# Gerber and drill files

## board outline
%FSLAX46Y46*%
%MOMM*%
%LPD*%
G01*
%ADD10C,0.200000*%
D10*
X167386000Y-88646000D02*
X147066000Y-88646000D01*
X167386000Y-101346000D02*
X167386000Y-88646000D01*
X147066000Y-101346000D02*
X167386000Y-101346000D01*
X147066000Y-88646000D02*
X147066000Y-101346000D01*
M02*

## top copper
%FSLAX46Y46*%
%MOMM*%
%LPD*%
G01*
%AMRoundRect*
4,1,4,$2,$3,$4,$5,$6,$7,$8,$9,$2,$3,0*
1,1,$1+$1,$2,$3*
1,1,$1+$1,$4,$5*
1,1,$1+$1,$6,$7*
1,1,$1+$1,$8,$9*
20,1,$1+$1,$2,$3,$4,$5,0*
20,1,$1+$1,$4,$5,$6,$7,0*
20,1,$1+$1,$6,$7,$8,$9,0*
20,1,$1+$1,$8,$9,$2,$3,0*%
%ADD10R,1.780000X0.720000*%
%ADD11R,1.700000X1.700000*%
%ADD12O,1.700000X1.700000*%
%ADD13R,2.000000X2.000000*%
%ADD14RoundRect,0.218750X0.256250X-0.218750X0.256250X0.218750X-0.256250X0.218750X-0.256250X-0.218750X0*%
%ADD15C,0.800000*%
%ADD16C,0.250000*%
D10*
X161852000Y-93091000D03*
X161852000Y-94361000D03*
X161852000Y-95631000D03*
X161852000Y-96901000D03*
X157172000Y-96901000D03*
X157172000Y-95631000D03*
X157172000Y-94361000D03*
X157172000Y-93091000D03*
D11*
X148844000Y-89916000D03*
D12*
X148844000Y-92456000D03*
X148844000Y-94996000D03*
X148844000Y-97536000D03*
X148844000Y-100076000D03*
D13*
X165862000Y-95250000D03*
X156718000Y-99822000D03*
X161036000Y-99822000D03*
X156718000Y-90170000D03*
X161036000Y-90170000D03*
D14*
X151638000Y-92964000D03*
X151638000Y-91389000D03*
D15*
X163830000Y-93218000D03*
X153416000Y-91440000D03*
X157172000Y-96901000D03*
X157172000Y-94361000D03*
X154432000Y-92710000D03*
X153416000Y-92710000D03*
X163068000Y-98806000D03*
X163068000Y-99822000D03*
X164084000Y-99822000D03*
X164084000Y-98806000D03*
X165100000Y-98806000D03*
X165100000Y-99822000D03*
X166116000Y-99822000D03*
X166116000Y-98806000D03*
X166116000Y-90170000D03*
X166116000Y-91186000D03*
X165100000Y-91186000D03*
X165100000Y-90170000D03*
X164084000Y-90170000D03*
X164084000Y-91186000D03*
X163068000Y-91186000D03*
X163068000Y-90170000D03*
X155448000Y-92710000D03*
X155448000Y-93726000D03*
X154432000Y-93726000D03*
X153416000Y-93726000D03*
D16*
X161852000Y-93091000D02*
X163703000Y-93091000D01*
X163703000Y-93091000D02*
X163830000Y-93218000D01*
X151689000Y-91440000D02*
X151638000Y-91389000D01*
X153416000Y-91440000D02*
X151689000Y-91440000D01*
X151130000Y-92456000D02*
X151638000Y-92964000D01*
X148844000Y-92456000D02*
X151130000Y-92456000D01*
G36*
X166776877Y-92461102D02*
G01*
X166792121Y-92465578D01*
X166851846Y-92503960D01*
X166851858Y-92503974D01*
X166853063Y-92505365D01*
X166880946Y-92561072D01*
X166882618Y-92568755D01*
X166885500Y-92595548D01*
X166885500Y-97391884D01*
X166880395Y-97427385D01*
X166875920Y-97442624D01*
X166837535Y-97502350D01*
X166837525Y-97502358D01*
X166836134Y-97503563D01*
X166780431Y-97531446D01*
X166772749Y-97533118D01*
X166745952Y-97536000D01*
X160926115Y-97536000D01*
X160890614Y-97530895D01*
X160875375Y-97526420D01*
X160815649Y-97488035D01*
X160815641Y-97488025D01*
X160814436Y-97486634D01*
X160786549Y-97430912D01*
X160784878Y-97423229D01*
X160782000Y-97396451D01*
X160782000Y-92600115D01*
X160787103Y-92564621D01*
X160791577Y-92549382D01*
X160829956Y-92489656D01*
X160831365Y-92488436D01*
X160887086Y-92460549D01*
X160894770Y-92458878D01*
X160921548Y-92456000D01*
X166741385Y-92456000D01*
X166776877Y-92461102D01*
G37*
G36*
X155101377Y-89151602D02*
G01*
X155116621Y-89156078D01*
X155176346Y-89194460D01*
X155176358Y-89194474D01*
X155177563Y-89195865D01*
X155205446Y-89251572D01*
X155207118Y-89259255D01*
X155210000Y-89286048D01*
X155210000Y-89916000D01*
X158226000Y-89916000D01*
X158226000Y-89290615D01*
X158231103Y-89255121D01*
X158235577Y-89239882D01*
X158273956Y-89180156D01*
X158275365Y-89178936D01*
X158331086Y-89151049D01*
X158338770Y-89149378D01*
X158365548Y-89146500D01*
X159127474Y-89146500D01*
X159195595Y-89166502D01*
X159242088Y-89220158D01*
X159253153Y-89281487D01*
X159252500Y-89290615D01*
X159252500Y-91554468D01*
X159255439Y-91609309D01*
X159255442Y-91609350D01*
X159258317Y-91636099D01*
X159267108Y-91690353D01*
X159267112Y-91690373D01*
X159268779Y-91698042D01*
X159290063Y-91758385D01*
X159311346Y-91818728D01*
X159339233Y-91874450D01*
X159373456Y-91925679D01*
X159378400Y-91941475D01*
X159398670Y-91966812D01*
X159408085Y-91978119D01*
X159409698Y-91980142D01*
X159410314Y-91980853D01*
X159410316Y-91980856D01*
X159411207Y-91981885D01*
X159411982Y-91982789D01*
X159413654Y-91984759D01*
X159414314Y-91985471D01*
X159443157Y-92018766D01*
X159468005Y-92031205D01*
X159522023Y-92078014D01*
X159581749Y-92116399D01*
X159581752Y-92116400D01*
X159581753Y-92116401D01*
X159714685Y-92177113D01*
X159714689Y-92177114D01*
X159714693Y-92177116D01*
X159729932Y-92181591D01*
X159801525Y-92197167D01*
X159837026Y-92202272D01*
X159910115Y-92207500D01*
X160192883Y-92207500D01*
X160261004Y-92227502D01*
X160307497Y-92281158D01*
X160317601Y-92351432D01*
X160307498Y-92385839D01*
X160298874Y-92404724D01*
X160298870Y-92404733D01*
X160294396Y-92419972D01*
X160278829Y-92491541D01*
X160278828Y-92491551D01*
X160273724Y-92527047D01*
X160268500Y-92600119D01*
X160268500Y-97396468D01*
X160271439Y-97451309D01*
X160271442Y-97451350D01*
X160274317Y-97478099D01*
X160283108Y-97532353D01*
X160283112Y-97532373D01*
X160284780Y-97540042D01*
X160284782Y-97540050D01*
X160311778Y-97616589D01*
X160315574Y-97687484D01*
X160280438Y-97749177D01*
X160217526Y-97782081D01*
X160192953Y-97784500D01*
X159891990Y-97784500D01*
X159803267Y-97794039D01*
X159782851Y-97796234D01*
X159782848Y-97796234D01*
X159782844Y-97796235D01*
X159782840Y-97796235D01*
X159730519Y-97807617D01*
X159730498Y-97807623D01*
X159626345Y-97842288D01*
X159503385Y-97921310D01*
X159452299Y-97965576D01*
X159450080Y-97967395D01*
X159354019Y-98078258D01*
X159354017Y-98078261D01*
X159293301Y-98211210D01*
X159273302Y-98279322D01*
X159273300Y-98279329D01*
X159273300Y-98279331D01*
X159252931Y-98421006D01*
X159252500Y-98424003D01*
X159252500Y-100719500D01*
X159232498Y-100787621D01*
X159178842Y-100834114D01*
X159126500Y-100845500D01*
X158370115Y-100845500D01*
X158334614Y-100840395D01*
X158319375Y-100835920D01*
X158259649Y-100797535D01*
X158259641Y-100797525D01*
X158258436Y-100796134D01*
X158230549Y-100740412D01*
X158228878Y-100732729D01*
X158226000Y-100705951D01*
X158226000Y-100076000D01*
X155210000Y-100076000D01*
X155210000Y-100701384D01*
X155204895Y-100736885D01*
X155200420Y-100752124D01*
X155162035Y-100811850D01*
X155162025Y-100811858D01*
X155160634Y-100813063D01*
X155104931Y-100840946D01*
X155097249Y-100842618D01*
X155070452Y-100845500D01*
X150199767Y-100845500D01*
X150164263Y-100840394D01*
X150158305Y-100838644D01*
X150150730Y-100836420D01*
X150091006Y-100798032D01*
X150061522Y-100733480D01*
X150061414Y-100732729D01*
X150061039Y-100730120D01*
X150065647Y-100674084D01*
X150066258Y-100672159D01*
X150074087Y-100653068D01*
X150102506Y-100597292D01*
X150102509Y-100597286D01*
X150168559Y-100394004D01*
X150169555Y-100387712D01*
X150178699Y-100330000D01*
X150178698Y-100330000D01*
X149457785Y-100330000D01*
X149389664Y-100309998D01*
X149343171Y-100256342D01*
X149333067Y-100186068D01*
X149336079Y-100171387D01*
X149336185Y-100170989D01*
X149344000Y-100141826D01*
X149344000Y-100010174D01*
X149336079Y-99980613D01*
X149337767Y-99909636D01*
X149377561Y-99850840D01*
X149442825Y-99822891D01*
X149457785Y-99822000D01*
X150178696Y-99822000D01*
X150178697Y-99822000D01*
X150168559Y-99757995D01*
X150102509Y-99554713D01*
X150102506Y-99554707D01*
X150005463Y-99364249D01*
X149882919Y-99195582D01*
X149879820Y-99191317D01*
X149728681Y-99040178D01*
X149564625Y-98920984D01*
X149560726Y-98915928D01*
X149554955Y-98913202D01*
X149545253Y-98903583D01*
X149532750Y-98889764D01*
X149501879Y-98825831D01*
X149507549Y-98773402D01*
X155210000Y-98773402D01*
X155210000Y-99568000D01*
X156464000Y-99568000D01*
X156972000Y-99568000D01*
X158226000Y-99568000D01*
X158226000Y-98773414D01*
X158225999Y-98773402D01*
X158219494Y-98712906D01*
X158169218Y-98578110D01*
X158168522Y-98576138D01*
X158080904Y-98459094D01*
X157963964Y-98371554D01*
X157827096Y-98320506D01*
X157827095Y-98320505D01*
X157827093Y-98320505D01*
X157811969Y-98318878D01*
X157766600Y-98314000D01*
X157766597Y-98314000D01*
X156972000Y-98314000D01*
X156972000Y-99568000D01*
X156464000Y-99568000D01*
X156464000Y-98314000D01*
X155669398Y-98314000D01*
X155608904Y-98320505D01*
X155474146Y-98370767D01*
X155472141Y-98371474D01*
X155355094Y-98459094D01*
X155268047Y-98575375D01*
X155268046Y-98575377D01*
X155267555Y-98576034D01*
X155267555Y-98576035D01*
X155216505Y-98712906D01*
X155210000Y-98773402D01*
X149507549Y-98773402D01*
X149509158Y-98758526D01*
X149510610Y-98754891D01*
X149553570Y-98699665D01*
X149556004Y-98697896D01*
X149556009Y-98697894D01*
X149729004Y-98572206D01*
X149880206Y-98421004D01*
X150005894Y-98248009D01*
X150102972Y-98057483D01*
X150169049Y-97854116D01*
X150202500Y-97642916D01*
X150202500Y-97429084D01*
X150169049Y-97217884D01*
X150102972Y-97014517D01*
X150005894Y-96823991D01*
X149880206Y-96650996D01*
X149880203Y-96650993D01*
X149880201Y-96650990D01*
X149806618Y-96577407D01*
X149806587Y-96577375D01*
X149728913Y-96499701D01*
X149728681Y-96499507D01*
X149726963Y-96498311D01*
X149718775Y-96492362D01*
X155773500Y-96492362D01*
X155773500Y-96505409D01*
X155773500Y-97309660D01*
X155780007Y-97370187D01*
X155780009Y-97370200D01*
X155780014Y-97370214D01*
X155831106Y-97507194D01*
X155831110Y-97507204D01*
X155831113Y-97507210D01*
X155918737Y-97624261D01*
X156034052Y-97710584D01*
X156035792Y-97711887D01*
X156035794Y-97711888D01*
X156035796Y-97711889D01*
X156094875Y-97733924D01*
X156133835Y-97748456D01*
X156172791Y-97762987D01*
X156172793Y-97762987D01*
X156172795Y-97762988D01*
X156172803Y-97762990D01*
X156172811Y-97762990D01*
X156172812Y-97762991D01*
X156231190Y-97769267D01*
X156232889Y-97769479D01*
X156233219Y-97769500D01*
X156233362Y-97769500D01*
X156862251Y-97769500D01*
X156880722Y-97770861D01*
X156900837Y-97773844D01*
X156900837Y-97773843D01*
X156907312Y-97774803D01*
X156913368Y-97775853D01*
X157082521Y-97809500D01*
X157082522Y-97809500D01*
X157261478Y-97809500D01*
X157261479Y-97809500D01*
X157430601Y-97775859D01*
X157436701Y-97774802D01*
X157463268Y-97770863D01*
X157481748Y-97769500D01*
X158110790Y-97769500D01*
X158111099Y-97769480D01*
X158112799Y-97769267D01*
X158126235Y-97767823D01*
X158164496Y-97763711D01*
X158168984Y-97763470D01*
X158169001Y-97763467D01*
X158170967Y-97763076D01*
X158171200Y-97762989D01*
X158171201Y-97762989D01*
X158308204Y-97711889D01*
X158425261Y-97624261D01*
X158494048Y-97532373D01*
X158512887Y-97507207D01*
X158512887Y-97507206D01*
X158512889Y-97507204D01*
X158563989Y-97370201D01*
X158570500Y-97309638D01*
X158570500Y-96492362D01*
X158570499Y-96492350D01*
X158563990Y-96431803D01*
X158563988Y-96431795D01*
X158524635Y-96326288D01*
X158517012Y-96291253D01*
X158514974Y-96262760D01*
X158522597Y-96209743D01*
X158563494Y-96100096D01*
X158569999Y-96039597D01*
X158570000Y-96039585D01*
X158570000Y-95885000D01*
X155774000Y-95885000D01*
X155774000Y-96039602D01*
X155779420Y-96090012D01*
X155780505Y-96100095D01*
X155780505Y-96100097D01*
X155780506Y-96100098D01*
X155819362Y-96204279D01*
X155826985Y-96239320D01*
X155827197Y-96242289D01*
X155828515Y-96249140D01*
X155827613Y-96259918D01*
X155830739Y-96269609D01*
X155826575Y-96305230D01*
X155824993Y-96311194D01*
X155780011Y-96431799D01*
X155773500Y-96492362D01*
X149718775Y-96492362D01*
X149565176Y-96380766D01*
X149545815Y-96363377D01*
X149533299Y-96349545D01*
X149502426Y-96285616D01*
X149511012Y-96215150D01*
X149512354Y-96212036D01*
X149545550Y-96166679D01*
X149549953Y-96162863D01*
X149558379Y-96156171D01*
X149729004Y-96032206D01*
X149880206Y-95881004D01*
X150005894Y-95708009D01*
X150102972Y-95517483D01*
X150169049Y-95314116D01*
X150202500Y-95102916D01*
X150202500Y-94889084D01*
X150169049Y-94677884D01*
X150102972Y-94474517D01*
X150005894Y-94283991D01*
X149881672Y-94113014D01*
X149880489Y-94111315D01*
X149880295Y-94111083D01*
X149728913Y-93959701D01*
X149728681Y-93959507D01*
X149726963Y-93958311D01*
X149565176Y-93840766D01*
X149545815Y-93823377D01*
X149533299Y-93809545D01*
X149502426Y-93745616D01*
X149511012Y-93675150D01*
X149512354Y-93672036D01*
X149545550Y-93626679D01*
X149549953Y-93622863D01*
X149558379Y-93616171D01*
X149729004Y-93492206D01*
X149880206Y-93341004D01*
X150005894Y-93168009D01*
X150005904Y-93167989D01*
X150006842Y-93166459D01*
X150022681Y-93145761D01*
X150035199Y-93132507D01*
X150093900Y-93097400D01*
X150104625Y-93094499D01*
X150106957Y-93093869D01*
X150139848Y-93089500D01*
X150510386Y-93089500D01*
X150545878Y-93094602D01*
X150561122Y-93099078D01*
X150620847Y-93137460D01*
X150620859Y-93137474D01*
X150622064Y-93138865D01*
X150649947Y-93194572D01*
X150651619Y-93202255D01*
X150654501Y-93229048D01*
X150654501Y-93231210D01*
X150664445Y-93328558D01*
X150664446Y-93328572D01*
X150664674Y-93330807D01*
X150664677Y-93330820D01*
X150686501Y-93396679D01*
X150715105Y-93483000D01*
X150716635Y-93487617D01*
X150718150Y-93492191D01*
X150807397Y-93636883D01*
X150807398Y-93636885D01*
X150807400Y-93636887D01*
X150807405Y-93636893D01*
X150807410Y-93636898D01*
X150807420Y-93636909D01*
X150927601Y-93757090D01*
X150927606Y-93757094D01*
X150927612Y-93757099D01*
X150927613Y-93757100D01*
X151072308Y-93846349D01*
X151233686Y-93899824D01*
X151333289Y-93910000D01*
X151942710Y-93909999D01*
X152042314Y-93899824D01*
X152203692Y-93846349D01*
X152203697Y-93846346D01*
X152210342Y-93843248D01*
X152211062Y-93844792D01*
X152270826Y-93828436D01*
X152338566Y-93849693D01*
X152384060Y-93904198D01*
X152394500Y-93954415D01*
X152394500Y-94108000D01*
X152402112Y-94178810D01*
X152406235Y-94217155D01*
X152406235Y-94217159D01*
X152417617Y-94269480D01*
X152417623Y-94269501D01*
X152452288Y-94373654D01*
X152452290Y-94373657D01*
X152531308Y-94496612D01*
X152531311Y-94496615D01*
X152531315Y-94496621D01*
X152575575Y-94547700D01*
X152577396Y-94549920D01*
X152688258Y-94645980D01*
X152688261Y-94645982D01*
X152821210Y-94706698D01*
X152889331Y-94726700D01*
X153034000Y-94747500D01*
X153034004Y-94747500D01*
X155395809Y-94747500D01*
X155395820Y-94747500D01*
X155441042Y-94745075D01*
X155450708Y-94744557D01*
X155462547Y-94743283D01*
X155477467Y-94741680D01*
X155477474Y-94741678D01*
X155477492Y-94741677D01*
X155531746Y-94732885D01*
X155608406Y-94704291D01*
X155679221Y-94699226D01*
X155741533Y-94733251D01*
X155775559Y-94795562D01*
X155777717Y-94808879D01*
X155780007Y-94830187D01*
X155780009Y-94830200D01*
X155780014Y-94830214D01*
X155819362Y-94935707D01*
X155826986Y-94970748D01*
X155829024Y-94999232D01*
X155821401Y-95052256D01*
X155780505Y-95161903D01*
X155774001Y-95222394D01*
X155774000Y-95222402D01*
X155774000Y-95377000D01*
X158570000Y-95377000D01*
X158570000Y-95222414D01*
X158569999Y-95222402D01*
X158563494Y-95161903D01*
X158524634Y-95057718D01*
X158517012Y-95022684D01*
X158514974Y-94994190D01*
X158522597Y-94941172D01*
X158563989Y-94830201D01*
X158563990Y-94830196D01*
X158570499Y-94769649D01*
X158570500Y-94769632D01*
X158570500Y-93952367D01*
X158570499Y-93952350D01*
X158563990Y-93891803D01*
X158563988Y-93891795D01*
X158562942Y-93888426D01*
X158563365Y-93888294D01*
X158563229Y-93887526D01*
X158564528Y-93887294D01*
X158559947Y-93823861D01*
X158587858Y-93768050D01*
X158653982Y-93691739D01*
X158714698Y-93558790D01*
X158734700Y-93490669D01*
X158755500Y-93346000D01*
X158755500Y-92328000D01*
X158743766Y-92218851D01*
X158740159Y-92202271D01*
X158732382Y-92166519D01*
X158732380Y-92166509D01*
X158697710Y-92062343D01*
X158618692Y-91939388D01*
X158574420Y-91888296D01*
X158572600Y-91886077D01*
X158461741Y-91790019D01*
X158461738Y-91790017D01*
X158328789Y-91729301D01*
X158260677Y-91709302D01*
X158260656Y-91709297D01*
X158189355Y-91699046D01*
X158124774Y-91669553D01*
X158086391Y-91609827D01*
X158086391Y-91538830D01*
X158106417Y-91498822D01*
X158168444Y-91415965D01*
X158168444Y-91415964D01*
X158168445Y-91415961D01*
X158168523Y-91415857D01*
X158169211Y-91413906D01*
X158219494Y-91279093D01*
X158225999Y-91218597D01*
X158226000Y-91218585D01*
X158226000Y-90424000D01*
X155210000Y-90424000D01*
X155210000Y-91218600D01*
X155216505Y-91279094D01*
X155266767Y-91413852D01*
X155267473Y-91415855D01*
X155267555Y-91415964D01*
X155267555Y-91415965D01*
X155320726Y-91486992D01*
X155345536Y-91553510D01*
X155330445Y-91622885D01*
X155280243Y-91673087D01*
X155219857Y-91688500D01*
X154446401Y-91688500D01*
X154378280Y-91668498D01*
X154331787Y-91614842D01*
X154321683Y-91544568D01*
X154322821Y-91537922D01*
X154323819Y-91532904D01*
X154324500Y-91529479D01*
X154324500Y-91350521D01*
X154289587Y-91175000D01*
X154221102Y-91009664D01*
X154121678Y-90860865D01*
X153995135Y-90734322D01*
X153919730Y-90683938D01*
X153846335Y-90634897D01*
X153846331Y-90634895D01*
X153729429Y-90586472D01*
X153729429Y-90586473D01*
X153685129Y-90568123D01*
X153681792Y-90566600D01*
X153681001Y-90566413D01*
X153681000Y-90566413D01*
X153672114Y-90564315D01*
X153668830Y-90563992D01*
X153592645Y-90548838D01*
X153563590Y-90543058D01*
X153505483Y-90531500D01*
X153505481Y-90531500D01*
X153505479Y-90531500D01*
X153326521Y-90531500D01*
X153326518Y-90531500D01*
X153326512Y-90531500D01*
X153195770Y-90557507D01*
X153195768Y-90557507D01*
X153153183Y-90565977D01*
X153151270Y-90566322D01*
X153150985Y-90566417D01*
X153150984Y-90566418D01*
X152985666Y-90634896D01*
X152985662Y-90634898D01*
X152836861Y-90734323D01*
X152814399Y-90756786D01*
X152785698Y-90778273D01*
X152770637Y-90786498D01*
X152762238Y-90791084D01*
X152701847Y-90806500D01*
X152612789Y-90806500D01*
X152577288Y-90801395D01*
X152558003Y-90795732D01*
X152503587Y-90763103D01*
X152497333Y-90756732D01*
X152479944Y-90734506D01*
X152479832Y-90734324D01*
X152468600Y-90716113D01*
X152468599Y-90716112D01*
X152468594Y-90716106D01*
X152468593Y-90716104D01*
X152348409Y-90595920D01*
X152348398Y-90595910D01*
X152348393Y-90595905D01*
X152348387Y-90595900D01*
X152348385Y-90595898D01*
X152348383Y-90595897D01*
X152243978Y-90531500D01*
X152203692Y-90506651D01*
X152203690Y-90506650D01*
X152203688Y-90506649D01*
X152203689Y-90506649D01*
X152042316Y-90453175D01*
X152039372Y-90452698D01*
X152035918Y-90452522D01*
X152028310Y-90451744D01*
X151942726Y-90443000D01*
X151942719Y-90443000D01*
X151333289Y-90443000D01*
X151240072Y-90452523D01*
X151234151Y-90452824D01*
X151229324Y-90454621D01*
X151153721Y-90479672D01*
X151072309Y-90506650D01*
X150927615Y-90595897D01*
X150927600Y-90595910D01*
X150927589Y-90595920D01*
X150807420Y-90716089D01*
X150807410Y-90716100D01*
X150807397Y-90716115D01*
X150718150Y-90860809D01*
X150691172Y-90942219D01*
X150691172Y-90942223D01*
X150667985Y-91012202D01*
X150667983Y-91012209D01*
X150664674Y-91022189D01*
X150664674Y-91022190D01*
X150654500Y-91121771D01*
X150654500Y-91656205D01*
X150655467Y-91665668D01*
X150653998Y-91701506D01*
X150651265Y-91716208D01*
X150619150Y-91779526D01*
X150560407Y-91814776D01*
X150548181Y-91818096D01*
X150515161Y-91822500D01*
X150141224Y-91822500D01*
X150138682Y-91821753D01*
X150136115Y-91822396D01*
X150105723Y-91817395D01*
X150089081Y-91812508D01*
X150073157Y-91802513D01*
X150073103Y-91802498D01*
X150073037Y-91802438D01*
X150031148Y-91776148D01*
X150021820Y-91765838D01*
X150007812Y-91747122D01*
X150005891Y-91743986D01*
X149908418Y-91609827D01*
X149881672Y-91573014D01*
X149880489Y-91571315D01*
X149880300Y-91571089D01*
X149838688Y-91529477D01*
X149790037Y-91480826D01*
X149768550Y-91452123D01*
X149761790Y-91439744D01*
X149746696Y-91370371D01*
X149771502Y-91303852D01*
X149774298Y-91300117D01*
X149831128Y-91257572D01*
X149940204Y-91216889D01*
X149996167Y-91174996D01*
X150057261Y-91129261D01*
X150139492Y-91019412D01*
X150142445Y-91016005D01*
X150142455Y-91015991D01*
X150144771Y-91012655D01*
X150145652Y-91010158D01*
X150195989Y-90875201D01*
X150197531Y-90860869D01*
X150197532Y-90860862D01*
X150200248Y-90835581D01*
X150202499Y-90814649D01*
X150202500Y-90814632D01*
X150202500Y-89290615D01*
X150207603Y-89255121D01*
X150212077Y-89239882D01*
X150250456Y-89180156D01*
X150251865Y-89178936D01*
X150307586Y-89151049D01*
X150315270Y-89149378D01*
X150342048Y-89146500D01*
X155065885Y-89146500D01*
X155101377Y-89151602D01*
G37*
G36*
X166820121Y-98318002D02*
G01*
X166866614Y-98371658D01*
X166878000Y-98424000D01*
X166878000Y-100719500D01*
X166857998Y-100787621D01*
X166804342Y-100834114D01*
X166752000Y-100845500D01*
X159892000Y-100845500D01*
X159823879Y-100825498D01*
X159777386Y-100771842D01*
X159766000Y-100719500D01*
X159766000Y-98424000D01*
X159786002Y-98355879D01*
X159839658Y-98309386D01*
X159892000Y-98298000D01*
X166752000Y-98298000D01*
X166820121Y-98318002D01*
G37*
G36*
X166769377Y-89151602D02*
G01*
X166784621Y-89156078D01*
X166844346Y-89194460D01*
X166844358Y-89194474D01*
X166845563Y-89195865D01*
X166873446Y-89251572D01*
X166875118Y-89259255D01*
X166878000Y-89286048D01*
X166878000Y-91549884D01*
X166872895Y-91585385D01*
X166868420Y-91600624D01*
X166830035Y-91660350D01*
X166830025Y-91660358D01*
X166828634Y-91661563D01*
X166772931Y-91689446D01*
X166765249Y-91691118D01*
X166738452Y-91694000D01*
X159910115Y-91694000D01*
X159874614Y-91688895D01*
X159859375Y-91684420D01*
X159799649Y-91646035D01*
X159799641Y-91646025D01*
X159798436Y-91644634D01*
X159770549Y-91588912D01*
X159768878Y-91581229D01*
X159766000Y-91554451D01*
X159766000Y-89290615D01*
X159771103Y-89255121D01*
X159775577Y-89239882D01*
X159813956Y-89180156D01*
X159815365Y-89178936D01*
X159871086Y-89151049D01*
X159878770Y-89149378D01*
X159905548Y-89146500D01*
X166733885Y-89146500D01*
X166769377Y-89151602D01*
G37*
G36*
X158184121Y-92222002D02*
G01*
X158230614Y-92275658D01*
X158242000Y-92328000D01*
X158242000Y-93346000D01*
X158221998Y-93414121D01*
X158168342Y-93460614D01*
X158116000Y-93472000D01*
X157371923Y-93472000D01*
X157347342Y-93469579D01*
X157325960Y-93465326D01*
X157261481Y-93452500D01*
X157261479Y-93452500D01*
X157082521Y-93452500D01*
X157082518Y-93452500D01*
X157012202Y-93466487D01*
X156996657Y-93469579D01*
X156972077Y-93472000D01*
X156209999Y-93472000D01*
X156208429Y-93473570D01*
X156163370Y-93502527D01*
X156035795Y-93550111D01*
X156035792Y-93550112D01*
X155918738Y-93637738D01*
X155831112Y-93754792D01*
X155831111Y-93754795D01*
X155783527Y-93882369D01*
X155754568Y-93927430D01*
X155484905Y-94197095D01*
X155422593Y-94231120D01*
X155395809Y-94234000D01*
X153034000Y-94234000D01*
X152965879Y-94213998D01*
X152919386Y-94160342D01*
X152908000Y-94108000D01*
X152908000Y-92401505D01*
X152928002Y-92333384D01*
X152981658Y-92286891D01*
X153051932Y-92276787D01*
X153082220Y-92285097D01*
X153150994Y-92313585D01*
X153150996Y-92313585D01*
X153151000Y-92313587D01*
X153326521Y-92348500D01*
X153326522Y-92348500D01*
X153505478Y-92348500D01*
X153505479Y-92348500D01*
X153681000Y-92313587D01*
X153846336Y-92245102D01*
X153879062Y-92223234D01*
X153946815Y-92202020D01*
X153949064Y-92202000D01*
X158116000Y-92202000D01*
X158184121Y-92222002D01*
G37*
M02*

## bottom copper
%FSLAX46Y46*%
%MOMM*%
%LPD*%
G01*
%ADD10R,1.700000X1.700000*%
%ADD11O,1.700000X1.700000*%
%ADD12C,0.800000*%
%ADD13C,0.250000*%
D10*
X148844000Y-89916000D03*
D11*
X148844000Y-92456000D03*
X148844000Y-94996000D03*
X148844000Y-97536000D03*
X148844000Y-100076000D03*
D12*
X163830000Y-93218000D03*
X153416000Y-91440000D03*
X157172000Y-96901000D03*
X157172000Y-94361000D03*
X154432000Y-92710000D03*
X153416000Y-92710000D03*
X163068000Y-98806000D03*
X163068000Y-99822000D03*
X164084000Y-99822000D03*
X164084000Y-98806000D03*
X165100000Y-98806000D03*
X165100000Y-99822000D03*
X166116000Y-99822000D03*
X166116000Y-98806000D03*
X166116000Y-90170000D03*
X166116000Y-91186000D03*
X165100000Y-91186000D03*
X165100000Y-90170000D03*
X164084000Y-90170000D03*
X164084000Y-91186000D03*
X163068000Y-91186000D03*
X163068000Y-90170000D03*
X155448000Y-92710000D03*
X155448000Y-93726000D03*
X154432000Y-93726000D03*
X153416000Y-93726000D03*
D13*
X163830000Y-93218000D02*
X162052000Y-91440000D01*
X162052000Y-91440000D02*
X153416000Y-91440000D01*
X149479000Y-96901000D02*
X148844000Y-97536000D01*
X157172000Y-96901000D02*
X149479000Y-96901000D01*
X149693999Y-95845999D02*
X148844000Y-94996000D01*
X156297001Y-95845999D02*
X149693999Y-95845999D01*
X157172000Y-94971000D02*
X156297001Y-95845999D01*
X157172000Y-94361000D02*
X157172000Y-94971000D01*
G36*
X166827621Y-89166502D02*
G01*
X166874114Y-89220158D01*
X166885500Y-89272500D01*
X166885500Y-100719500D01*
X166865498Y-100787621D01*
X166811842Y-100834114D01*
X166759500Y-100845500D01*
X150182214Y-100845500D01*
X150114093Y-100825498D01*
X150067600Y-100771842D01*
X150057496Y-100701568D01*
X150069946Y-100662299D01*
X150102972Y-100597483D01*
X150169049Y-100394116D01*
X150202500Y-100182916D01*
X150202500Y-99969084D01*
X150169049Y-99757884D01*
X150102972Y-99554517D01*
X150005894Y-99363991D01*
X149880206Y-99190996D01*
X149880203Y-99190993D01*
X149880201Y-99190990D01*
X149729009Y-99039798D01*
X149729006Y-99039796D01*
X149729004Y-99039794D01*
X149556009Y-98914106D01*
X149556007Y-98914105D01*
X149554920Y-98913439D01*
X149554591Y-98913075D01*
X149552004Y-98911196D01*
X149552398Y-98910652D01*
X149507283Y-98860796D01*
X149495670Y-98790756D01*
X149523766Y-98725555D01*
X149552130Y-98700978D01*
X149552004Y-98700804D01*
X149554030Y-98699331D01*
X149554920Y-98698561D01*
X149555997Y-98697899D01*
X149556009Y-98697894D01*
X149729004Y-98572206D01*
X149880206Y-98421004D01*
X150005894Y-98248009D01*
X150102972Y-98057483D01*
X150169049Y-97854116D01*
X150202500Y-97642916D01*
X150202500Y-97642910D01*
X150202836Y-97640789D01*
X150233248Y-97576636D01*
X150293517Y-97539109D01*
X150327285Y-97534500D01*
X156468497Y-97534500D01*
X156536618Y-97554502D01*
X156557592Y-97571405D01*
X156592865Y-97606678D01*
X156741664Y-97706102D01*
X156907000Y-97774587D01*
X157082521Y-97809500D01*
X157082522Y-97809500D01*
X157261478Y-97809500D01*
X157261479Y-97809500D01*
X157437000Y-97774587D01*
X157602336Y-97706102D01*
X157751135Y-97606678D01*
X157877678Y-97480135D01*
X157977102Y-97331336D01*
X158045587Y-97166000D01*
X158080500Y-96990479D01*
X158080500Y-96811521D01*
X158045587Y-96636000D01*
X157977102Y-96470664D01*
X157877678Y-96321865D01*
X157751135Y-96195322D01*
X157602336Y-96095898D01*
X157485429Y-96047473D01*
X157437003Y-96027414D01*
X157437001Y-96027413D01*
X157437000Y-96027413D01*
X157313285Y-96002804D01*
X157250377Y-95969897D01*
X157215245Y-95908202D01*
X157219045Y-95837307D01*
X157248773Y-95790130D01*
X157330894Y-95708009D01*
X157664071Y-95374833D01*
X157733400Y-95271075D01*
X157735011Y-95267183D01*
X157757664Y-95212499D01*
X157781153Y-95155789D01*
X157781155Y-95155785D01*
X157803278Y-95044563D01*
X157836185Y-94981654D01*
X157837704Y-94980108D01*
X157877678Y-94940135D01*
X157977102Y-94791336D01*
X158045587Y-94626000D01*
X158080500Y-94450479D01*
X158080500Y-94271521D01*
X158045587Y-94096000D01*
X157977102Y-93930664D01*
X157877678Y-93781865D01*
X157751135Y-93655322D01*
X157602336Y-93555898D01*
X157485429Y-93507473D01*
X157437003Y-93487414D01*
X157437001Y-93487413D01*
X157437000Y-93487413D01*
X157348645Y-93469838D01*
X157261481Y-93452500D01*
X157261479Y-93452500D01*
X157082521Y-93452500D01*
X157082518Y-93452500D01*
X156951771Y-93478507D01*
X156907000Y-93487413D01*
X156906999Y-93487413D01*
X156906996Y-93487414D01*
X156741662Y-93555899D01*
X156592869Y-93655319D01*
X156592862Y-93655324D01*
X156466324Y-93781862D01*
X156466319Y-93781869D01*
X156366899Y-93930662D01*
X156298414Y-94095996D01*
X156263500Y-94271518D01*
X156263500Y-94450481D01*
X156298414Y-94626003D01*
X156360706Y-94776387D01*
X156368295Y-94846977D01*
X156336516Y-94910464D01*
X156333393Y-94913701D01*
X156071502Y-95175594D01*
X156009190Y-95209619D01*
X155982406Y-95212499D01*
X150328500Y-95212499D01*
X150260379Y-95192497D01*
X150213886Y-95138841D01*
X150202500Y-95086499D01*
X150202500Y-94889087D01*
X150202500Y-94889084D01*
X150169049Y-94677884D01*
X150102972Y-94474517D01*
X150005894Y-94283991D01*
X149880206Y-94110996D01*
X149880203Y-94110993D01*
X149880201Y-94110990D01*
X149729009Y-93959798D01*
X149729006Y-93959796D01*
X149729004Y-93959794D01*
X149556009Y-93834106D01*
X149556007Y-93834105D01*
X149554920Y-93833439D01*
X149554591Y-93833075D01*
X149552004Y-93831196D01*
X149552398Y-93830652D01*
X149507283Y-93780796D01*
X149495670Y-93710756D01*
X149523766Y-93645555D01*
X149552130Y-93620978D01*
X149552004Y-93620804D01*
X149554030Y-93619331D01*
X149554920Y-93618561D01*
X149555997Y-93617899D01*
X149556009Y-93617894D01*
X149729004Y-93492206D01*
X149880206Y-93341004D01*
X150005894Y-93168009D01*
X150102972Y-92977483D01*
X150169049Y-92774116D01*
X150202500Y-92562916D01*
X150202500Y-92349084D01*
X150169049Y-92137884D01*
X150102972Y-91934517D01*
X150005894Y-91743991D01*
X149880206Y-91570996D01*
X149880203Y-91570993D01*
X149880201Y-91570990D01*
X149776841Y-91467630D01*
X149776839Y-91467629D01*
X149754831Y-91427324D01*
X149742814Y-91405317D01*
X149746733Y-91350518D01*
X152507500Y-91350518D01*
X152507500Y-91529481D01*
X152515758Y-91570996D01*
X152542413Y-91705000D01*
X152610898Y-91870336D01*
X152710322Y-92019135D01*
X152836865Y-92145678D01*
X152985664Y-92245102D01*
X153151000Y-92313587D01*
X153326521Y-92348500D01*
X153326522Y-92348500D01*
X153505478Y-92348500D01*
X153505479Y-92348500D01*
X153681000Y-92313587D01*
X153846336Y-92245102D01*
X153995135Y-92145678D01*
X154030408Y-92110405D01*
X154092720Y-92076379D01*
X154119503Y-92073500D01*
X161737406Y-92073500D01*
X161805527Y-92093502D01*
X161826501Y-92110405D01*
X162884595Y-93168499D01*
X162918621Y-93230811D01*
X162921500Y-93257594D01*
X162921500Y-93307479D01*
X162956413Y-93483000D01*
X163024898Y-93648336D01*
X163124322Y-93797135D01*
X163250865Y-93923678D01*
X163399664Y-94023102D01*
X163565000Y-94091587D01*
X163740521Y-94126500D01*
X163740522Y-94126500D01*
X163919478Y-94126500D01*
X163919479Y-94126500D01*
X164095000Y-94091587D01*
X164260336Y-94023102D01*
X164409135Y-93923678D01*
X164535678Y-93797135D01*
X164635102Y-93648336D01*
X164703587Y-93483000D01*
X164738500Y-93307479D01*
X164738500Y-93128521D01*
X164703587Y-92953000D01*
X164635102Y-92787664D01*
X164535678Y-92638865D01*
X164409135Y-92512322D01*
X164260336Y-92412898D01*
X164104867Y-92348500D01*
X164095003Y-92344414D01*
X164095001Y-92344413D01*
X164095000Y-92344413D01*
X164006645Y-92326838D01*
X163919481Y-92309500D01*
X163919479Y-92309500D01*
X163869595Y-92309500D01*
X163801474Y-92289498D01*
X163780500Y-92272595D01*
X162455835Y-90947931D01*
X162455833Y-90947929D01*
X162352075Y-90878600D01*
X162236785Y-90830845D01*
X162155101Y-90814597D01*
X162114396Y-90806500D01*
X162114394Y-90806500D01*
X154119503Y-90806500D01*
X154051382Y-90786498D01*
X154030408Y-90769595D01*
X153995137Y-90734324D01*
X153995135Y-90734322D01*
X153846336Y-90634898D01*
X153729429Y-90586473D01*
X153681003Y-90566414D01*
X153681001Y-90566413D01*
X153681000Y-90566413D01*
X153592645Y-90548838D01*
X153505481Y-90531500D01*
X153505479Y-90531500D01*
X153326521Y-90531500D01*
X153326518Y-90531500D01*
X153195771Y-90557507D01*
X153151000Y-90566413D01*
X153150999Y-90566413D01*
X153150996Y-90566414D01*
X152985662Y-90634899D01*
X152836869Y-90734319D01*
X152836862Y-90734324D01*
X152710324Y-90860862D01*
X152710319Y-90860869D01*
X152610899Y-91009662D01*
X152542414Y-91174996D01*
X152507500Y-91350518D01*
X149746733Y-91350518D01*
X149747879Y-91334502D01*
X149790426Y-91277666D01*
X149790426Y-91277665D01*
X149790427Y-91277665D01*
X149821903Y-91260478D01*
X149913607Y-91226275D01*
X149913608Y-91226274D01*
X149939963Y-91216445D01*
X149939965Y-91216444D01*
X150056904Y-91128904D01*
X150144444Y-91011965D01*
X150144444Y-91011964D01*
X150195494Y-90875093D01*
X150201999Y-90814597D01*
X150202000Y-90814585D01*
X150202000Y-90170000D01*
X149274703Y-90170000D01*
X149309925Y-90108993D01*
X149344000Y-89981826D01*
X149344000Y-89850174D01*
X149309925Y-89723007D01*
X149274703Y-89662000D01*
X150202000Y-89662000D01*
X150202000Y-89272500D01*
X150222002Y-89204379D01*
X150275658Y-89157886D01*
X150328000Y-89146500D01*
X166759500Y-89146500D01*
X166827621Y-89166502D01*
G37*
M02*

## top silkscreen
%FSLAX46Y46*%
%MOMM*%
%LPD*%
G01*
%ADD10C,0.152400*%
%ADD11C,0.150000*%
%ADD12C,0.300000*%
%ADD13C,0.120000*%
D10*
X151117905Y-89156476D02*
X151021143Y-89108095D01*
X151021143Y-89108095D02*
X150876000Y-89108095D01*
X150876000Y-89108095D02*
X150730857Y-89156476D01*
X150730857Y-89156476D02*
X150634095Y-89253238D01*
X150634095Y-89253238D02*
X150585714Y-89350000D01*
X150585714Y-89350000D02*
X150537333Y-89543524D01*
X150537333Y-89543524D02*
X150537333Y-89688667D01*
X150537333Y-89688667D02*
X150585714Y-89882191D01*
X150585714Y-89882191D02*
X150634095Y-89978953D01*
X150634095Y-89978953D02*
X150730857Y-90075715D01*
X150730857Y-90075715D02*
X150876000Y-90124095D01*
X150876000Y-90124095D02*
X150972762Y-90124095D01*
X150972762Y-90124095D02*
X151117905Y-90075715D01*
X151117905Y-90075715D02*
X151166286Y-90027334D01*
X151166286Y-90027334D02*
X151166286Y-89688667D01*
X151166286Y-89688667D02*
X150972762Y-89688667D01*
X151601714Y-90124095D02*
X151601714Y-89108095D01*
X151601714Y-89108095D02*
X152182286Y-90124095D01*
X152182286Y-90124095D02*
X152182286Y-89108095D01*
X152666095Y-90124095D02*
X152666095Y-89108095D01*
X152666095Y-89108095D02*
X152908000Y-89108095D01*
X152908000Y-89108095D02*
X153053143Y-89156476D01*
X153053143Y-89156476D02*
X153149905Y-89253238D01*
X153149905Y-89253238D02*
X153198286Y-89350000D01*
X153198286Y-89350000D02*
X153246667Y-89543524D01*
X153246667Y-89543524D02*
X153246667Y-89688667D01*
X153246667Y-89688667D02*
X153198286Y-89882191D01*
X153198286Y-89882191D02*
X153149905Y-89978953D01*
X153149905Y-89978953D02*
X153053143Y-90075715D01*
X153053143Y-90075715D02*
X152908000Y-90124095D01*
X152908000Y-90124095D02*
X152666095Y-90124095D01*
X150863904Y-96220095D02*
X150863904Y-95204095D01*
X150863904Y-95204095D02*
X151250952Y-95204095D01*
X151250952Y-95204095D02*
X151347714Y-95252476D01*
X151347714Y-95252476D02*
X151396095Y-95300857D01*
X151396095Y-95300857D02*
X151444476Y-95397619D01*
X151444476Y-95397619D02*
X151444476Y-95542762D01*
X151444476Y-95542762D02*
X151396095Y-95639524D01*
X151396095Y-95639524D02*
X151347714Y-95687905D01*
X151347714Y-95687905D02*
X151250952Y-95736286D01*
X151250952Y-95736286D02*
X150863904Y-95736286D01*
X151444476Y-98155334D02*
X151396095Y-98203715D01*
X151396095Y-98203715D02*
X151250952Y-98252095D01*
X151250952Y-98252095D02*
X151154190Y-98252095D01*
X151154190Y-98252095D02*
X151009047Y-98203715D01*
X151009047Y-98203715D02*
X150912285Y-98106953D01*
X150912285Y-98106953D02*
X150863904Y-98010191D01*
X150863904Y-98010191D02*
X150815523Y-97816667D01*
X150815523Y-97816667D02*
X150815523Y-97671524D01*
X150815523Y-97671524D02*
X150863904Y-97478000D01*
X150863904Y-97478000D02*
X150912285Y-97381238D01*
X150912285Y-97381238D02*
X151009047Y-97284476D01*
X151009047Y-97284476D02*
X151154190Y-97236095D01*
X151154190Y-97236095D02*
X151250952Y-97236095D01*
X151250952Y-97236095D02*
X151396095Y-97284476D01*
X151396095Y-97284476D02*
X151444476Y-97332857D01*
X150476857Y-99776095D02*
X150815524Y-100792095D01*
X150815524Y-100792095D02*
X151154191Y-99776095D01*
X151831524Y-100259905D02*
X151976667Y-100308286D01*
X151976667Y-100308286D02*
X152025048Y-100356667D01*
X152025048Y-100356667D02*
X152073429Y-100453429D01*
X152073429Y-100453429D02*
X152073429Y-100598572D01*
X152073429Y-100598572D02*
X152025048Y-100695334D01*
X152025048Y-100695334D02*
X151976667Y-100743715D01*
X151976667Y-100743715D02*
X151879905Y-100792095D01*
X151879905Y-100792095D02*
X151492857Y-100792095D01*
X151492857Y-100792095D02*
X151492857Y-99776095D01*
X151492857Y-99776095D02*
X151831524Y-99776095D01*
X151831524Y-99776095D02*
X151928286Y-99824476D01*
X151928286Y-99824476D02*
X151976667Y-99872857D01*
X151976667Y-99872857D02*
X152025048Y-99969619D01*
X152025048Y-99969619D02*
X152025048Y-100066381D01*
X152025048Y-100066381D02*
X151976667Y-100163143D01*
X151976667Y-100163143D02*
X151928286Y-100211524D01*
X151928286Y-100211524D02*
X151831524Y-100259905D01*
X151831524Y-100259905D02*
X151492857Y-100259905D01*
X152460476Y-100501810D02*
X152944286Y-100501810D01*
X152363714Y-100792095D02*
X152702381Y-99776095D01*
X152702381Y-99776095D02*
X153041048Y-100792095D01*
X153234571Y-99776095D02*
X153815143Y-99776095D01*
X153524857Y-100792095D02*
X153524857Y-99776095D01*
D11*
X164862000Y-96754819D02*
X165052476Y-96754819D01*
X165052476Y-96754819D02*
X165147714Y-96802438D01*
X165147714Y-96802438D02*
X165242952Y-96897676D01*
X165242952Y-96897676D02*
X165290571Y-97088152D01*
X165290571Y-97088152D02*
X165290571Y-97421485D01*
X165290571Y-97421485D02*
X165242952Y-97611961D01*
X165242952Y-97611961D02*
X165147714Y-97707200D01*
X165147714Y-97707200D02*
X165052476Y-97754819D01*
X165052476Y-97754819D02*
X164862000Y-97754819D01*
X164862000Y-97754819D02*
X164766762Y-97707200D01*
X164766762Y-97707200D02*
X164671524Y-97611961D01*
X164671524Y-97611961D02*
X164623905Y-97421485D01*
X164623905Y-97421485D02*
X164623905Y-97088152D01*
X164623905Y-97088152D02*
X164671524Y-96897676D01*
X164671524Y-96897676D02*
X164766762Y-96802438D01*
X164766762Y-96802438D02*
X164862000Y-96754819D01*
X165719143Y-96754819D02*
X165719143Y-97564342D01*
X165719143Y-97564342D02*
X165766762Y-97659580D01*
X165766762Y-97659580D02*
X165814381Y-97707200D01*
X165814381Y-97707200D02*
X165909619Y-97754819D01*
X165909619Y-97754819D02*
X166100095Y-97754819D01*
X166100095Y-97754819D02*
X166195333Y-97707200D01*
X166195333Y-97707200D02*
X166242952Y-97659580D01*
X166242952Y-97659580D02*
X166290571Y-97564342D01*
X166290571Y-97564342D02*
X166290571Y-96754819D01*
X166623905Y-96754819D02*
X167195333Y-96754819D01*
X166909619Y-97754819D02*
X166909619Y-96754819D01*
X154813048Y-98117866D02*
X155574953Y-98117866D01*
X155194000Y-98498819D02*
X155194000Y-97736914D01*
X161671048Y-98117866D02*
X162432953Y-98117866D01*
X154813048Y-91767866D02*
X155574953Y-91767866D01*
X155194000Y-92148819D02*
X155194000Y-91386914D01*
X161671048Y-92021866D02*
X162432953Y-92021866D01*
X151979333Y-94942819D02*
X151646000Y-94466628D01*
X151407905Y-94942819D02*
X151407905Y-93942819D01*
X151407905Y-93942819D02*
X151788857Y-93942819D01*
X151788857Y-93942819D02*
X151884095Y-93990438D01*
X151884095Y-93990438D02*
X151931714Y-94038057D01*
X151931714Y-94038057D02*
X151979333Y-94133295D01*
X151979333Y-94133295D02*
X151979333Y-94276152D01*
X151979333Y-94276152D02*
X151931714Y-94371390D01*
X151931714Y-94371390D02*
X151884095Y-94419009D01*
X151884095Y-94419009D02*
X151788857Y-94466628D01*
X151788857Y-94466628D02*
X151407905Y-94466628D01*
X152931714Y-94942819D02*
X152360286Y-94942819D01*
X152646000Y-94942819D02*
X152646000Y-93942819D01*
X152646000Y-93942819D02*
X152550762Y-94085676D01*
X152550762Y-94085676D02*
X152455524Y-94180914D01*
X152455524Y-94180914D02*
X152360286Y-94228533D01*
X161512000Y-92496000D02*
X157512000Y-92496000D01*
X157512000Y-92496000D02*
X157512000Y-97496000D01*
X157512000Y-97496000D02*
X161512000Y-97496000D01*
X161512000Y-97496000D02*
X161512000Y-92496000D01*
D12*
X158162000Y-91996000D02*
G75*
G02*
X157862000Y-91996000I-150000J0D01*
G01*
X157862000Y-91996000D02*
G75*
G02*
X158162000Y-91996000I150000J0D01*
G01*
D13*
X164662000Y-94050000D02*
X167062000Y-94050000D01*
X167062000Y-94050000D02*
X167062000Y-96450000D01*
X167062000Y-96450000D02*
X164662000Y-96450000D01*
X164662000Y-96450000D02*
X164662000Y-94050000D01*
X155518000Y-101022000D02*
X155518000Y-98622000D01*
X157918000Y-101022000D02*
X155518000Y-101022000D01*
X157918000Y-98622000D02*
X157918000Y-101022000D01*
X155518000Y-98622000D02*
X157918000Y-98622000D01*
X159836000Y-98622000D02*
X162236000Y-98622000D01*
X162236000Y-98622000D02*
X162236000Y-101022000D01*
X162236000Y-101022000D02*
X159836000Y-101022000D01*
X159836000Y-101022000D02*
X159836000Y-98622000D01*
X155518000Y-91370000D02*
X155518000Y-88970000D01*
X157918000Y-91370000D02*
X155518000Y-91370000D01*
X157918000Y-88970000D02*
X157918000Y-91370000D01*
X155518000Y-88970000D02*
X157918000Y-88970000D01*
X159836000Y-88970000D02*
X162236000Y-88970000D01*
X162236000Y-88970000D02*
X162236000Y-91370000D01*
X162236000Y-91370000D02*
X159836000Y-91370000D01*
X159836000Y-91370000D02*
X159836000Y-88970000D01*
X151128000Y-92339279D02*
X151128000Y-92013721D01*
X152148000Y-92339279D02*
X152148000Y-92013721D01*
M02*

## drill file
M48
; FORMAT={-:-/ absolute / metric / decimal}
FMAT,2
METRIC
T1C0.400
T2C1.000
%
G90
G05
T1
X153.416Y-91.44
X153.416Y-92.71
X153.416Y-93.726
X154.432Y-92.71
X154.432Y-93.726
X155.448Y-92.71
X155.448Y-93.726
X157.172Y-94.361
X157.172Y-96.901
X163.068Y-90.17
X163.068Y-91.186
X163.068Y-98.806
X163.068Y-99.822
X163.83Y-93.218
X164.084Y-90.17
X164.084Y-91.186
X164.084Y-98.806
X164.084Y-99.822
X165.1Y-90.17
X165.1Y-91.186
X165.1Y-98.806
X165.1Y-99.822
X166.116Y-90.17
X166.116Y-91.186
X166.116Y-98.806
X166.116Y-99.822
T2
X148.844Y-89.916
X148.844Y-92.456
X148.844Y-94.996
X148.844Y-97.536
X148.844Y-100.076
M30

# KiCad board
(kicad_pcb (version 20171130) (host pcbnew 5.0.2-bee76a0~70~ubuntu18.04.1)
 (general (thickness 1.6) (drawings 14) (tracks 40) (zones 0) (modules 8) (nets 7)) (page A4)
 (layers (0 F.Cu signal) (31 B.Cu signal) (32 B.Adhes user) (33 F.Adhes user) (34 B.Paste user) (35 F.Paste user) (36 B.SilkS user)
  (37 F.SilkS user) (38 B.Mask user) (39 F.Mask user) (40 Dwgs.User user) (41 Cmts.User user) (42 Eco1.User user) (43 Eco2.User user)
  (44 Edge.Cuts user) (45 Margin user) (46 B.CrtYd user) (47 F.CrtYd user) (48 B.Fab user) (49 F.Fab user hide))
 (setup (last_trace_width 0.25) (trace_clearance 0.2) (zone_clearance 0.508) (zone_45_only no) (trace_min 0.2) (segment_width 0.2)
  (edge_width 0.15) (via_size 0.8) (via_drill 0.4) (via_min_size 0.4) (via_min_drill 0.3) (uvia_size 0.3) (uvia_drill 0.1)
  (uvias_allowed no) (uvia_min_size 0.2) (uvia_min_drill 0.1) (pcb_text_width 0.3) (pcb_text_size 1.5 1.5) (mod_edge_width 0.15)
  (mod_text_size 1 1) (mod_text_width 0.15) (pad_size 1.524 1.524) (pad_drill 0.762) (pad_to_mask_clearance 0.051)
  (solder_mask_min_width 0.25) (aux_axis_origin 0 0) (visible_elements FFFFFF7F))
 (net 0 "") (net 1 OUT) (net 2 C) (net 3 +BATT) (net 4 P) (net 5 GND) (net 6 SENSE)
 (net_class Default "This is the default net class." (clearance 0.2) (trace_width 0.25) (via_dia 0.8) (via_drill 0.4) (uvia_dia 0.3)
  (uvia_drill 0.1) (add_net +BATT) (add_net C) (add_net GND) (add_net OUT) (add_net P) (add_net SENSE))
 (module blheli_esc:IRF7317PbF (layer F.Cu) (at 159.512 94.996 270)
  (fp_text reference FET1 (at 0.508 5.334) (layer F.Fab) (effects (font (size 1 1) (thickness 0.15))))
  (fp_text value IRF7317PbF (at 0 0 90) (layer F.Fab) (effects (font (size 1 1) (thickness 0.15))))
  (fp_line (start -2.5 -2) (end -2.5 2) (layer F.SilkS) (width 0.15))
  (fp_line (start -2.5 2) (end 2.5 2) (layer F.SilkS) (width 0.15))
  (fp_line (start 2.5 2) (end 2.5 -2) (layer F.SilkS) (width 0.15))
  (fp_line (start 2.5 -2) (end -2.5 -2) (layer F.SilkS) (width 0.15))
  (fp_circle (center -3 1.5) (end -2.85 1.5) (layer F.SilkS) (width 0.3))
  (pad 8 smd rect (at -1.905 -2.34 270) (size 0.72 1.78) (layers F.Cu F.Paste F.Mask) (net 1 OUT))
  (pad 7 smd rect (at -0.635 -2.34 270) (size 0.72 1.78) (layers F.Cu F.Paste F.Mask) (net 1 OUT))
  (pad 6 smd rect (at 0.635 -2.34 270) (size 0.72 1.78) (layers F.Cu F.Paste F.Mask) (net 1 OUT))
  (pad 5 smd rect (at 1.905 -2.34 270) (size 0.72 1.78) (layers F.Cu F.Paste F.Mask) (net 1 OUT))
  (pad 4 smd rect (at 1.905 2.34 270) (size 0.72 1.78) (layers F.Cu F.Paste F.Mask) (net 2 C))
  (pad 3 smd rect (at 0.635 2.34 270) (size 0.72 1.78) (layers F.Cu F.Paste F.Mask) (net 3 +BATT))
  (pad 2 smd rect (at -0.635 2.34 270) (size 0.72 1.78) (layers F.Cu F.Paste F.Mask) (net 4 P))
  (pad 1 smd rect (at -1.905 2.34 270) (size 0.72 1.78) (layers F.Cu F.Paste F.Mask) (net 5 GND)))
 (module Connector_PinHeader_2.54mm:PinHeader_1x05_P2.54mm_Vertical (layer B.Cu) (at 148.844 89.916 180)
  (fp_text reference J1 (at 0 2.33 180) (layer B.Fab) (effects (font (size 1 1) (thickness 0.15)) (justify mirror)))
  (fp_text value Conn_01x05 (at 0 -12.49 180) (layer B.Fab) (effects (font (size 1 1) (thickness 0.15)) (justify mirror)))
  (pad 1 thru_hole rect (at 0 0 180) (size 1.7 1.7) (drill 1) (layers *.Cu *.Mask) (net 5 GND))
  (pad 2 thru_hole oval (at 0 -2.54 180) (size 1.7 1.7) (drill 1) (layers *.Cu *.Mask) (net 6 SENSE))
  (pad 3 thru_hole oval (at 0 -5.08 180) (size 1.7 1.7) (drill 1) (layers *.Cu *.Mask) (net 4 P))
  (pad 4 thru_hole oval (at 0 -7.62 180) (size 1.7 1.7) (drill 1) (layers *.Cu *.Mask) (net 2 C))
  (pad 5 thru_hole oval (at 0 -10.16 180) (size 1.7 1.7) (drill 1) (layers *.Cu *.Mask) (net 3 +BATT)))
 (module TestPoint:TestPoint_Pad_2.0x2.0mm (layer F.Cu) (at 165.862 95.25)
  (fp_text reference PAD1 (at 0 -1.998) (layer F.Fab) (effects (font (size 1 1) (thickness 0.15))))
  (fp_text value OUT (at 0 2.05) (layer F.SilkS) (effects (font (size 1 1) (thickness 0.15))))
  (fp_line (start -1.2 -1.2) (end 1.2 -1.2) (layer F.SilkS) (width 0.12))
  (fp_line (start 1.2 -1.2) (end 1.2 1.2) (layer F.SilkS) (width 0.12))
  (fp_line (start 1.2 1.2) (end -1.2 1.2) (layer F.SilkS) (width 0.12))
  (fp_line (start -1.2 1.2) (end -1.2 -1.2) (layer F.SilkS) (width 0.12))
  (pad 1 smd rect (at 0 0) (size 2 2) (layers F.Cu F.Mask) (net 1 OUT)))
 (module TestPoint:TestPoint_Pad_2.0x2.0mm (layer F.Cu) (at 156.718 99.822)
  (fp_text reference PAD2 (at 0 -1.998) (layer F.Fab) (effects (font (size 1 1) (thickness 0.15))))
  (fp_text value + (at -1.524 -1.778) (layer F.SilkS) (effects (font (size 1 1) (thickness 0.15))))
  (fp_line (start -1.2 1.2) (end -1.2 -1.2) (layer F.SilkS) (width 0.12))
  (fp_line (start 1.2 1.2) (end -1.2 1.2) (layer F.SilkS) (width 0.12))
  (fp_line (start 1.2 -1.2) (end 1.2 1.2) (layer F.SilkS) (width 0.12))
  (fp_line (start -1.2 -1.2) (end 1.2 -1.2) (layer F.SilkS) (width 0.12))
  (pad 1 smd rect (at 0 0) (size 2 2) (layers F.Cu F.Mask) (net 3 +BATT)))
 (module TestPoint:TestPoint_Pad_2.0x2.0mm (layer F.Cu) (at 161.036 99.822)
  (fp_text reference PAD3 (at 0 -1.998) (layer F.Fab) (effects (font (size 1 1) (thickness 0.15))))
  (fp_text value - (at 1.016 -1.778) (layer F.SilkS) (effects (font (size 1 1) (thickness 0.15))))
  (fp_line (start -1.2 -1.2) (end 1.2 -1.2) (layer F.SilkS) (width 0.12))
  (fp_line (start 1.2 -1.2) (end 1.2 1.2) (layer F.SilkS) (width 0.12))
  (fp_line (start 1.2 1.2) (end -1.2 1.2) (layer F.SilkS) (width 0.12))
  (fp_line (start -1.2 1.2) (end -1.2 -1.2) (layer F.SilkS) (width 0.12))
  (pad 1 smd rect (at 0 0) (size 2 2) (layers F.Cu F.Mask) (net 5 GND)))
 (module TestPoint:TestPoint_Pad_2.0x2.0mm (layer F.Cu) (at 156.718 90.17)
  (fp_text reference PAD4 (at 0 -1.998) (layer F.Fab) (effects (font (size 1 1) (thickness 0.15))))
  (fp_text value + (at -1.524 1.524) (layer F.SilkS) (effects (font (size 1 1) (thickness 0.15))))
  (fp_line (start -1.2 1.2) (end -1.2 -1.2) (layer F.SilkS) (width 0.12))
  (fp_line (start 1.2 1.2) (end -1.2 1.2) (layer F.SilkS) (width 0.12))
  (fp_line (start 1.2 -1.2) (end 1.2 1.2) (layer F.SilkS) (width 0.12))
  (fp_line (start -1.2 -1.2) (end 1.2 -1.2) (layer F.SilkS) (width 0.12))
  (pad 1 smd rect (at 0 0) (size 2 2) (layers F.Cu F.Mask) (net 3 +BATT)))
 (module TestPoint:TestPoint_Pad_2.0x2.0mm (layer F.Cu) (at 161.036 90.17)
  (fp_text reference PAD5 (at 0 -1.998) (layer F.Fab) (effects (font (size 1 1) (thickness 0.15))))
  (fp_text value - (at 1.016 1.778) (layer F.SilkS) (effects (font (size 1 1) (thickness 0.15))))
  (fp_line (start -1.2 -1.2) (end 1.2 -1.2) (layer F.SilkS) (width 0.12))
  (fp_line (start 1.2 -1.2) (end 1.2 1.2) (layer F.SilkS) (width 0.12))
  (fp_line (start 1.2 1.2) (end -1.2 1.2) (layer F.SilkS) (width 0.12))
  (fp_line (start -1.2 1.2) (end -1.2 -1.2) (layer F.SilkS) (width 0.12))
  (pad 1 smd rect (at 0 0) (size 2 2) (layers F.Cu F.Mask) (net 5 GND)))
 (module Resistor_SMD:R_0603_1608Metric (layer F.Cu) (at 151.638 92.1765 90)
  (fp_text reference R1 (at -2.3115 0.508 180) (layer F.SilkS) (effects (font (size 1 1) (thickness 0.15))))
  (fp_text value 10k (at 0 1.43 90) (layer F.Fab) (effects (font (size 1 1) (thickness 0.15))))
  (fp_line (start -0.162779 -0.51) (end 0.162779 -0.51) (layer F.SilkS) (width 0.12))
  (fp_line (start -0.162779 0.51) (end 0.162779 0.51) (layer F.SilkS) (width 0.12))
  (pad 1 smd roundrect (at -0.7875 0 90) (size 0.875 0.95) (layers F.Cu F.Paste F.Mask) (roundrect_rratio 0.25) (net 6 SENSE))
  (pad 2 smd roundrect (at 0.7875 0 90) (size 0.875 0.95) (layers F.Cu F.Paste F.Mask) (roundrect_rratio 0.25) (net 1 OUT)))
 (gr_line (start 167.386 88.646) (end 147.066 88.646) (layer Edge.Cuts) (width 0.2))
 (gr_line (start 167.386 101.346) (end 167.386 88.646) (layer Edge.Cuts) (width 0.2))
 (gr_line (start 147.066 101.346) (end 167.386 101.346) (layer Edge.Cuts) (width 0.2))
 (gr_line (start 147.066 88.646) (end 147.066 101.346) (layer Edge.Cuts) (width 0.2))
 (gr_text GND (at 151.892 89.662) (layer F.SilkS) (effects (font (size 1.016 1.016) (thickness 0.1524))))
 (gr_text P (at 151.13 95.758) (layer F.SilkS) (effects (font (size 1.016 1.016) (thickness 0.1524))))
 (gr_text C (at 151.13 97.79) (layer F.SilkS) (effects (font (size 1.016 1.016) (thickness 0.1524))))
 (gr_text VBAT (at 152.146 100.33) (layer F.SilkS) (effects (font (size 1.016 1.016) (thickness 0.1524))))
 (via (at 163.83 93.218) (size 0.8) (drill 0.4) (layers F.Cu B.Cu) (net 1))
 (segment (start 161.852 93.091) (end 163.703 93.091) (width 0.25) (layer F.Cu) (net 1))
 (segment (start 163.703 93.091) (end 163.83 93.218) (width 0.25) (layer F.Cu) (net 1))
 (via (at 153.416 91.44) (size 0.8) (drill 0.4) (layers F.Cu B.Cu) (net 1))
 (segment (start 163.83 93.218) (end 162.052 91.44) (width 0.25) (layer B.Cu) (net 1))
 (segment (start 162.052 91.44) (end 153.416 91.44) (width 0.25) (layer B.Cu) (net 1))
 (segment (start 151.689 91.44) (end 151.638 91.389) (width 0.25) (layer F.Cu) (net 1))
 (segment (start 153.416 91.44) (end 151.689 91.44) (width 0.25) (layer F.Cu) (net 1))
 (via (at 157.172 96.901) (size 0.8) (drill 0.4) (layers F.Cu B.Cu) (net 2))
 (segment (start 149.479 96.901) (end 148.844 97.536) (width 0.25) (layer B.Cu) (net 2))
 (segment (start 157.172 96.901) (end 149.479 96.901) (width 0.25) (layer B.Cu) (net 2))
 (via (at 157.172 94.361) (size 0.8) (drill 0.4) (layers F.Cu B.Cu) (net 4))
 (segment (start 149.693999 95.845999) (end 148.844 94.996) (width 0.25) (layer B.Cu) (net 4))
 (segment (start 156.297001 95.845999) (end 149.693999 95.845999) (width 0.25) (layer B.Cu) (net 4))
 (segment (start 157.172 94.971) (end 156.297001 95.845999) (width 0.25) (layer B.Cu) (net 4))
 (segment (start 157.172 94.361) (end 157.172 94.971) (width 0.25) (layer B.Cu) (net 4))
 (via (at 154.432 92.71) (size 0.8) (drill 0.4) (layers F.Cu B.Cu) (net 5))
 (via (at 153.416 92.71) (size 0.8) (drill 0.4) (layers F.Cu B.Cu) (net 5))
 (via (at 163.068 98.806) (size 0.8) (drill 0.4) (layers F.Cu B.Cu) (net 5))
 (via (at 163.068 99.822) (size 0.8) (drill 0.4) (layers F.Cu B.Cu) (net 5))
 (via (at 164.084 99.822) (size 0.8) (drill 0.4) (layers F.Cu B.Cu) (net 5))
 (via (at 164.084 98.806) (size 0.8) (drill 0.4) (layers F.Cu B.Cu) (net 5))
 (via (at 165.1 98.806) (size 0.8) (drill 0.4) (layers F.Cu B.Cu) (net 5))
 (via (at 165.1 99.822) (size 0.8) (drill 0.4) (layers F.Cu B.Cu) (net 5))
 (via (at 166.116 99.822) (size 0.8) (drill 0.4) (layers F.Cu B.Cu) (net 5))
 (via (at 166.116 98.806) (size 0.8) (drill 0.4) (layers F.Cu B.Cu) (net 5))
 (via (at 166.116 90.17) (size 0.8) (drill 0.4) (layers F.Cu B.Cu) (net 5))
 (via (at 166.116 91.186) (size 0.8) (drill 0.4) (layers F.Cu B.Cu) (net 5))
 (via (at 165.1 91.186) (size 0.8) (drill 0.4) (layers F.Cu B.Cu) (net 5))
 (via (at 165.1 90.17) (size 0.8) (drill 0.4) (layers F.Cu B.Cu) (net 5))
 (via (at 164.084 90.17) (size 0.8) (drill 0.4) (layers F.Cu B.Cu) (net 5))
 (via (at 164.084 91.186) (size 0.8) (drill 0.4) (layers F.Cu B.Cu) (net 5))
 (via (at 163.068 91.186) (size 0.8) (drill 0.4) (layers F.Cu B.Cu) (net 5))
 (via (at 163.068 90.17) (size 0.8) (drill 0.4) (layers F.Cu B.Cu) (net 5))
 (via (at 155.448 92.71) (size 0.8) (drill 0.4) (layers F.Cu B.Cu) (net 5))
 (via (at 155.448 93.726) (size 0.8) (drill 0.4) (layers F.Cu B.Cu) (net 5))
 (via (at 154.432 93.726) (size 0.8) (drill 0.4) (layers F.Cu B.Cu) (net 5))
 (via (at 153.416 93.726) (size 0.8) (drill 0.4) (layers F.Cu B.Cu) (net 5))
 (segment (start 151.13 92.456) (end 151.638 92.964) (width 0.25) (layer F.Cu) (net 6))
 (segment (start 148.844 92.456) (end 151.13 92.456) (width 0.25) (layer F.Cu) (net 6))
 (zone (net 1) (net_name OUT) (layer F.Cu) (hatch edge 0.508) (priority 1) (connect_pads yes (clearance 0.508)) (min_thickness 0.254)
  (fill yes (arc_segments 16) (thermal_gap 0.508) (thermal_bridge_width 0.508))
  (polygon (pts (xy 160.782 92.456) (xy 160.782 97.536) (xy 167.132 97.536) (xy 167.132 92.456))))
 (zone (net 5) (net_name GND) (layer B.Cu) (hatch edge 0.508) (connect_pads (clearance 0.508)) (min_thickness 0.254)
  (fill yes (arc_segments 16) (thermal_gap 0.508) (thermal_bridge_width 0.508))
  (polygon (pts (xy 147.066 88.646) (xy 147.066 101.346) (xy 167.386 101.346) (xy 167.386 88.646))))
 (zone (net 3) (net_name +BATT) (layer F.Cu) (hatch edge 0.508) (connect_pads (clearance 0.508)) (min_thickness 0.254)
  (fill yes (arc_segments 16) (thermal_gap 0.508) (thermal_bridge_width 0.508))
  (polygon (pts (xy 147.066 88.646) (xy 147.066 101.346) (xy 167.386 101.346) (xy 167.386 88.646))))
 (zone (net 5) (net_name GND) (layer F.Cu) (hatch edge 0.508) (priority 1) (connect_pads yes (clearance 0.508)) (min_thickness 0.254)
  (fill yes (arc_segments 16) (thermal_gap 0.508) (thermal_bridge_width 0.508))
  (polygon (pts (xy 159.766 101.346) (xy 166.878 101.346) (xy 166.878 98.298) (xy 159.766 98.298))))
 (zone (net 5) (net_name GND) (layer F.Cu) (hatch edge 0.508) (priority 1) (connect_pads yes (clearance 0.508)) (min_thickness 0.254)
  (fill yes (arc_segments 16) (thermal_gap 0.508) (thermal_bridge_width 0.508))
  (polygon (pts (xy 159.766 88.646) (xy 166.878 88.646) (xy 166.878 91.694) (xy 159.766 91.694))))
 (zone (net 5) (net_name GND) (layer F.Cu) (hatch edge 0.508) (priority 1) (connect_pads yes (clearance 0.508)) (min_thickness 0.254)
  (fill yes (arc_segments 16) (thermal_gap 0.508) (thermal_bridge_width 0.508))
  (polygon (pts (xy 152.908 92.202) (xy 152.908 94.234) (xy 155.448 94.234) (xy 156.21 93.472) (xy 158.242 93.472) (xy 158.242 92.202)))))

